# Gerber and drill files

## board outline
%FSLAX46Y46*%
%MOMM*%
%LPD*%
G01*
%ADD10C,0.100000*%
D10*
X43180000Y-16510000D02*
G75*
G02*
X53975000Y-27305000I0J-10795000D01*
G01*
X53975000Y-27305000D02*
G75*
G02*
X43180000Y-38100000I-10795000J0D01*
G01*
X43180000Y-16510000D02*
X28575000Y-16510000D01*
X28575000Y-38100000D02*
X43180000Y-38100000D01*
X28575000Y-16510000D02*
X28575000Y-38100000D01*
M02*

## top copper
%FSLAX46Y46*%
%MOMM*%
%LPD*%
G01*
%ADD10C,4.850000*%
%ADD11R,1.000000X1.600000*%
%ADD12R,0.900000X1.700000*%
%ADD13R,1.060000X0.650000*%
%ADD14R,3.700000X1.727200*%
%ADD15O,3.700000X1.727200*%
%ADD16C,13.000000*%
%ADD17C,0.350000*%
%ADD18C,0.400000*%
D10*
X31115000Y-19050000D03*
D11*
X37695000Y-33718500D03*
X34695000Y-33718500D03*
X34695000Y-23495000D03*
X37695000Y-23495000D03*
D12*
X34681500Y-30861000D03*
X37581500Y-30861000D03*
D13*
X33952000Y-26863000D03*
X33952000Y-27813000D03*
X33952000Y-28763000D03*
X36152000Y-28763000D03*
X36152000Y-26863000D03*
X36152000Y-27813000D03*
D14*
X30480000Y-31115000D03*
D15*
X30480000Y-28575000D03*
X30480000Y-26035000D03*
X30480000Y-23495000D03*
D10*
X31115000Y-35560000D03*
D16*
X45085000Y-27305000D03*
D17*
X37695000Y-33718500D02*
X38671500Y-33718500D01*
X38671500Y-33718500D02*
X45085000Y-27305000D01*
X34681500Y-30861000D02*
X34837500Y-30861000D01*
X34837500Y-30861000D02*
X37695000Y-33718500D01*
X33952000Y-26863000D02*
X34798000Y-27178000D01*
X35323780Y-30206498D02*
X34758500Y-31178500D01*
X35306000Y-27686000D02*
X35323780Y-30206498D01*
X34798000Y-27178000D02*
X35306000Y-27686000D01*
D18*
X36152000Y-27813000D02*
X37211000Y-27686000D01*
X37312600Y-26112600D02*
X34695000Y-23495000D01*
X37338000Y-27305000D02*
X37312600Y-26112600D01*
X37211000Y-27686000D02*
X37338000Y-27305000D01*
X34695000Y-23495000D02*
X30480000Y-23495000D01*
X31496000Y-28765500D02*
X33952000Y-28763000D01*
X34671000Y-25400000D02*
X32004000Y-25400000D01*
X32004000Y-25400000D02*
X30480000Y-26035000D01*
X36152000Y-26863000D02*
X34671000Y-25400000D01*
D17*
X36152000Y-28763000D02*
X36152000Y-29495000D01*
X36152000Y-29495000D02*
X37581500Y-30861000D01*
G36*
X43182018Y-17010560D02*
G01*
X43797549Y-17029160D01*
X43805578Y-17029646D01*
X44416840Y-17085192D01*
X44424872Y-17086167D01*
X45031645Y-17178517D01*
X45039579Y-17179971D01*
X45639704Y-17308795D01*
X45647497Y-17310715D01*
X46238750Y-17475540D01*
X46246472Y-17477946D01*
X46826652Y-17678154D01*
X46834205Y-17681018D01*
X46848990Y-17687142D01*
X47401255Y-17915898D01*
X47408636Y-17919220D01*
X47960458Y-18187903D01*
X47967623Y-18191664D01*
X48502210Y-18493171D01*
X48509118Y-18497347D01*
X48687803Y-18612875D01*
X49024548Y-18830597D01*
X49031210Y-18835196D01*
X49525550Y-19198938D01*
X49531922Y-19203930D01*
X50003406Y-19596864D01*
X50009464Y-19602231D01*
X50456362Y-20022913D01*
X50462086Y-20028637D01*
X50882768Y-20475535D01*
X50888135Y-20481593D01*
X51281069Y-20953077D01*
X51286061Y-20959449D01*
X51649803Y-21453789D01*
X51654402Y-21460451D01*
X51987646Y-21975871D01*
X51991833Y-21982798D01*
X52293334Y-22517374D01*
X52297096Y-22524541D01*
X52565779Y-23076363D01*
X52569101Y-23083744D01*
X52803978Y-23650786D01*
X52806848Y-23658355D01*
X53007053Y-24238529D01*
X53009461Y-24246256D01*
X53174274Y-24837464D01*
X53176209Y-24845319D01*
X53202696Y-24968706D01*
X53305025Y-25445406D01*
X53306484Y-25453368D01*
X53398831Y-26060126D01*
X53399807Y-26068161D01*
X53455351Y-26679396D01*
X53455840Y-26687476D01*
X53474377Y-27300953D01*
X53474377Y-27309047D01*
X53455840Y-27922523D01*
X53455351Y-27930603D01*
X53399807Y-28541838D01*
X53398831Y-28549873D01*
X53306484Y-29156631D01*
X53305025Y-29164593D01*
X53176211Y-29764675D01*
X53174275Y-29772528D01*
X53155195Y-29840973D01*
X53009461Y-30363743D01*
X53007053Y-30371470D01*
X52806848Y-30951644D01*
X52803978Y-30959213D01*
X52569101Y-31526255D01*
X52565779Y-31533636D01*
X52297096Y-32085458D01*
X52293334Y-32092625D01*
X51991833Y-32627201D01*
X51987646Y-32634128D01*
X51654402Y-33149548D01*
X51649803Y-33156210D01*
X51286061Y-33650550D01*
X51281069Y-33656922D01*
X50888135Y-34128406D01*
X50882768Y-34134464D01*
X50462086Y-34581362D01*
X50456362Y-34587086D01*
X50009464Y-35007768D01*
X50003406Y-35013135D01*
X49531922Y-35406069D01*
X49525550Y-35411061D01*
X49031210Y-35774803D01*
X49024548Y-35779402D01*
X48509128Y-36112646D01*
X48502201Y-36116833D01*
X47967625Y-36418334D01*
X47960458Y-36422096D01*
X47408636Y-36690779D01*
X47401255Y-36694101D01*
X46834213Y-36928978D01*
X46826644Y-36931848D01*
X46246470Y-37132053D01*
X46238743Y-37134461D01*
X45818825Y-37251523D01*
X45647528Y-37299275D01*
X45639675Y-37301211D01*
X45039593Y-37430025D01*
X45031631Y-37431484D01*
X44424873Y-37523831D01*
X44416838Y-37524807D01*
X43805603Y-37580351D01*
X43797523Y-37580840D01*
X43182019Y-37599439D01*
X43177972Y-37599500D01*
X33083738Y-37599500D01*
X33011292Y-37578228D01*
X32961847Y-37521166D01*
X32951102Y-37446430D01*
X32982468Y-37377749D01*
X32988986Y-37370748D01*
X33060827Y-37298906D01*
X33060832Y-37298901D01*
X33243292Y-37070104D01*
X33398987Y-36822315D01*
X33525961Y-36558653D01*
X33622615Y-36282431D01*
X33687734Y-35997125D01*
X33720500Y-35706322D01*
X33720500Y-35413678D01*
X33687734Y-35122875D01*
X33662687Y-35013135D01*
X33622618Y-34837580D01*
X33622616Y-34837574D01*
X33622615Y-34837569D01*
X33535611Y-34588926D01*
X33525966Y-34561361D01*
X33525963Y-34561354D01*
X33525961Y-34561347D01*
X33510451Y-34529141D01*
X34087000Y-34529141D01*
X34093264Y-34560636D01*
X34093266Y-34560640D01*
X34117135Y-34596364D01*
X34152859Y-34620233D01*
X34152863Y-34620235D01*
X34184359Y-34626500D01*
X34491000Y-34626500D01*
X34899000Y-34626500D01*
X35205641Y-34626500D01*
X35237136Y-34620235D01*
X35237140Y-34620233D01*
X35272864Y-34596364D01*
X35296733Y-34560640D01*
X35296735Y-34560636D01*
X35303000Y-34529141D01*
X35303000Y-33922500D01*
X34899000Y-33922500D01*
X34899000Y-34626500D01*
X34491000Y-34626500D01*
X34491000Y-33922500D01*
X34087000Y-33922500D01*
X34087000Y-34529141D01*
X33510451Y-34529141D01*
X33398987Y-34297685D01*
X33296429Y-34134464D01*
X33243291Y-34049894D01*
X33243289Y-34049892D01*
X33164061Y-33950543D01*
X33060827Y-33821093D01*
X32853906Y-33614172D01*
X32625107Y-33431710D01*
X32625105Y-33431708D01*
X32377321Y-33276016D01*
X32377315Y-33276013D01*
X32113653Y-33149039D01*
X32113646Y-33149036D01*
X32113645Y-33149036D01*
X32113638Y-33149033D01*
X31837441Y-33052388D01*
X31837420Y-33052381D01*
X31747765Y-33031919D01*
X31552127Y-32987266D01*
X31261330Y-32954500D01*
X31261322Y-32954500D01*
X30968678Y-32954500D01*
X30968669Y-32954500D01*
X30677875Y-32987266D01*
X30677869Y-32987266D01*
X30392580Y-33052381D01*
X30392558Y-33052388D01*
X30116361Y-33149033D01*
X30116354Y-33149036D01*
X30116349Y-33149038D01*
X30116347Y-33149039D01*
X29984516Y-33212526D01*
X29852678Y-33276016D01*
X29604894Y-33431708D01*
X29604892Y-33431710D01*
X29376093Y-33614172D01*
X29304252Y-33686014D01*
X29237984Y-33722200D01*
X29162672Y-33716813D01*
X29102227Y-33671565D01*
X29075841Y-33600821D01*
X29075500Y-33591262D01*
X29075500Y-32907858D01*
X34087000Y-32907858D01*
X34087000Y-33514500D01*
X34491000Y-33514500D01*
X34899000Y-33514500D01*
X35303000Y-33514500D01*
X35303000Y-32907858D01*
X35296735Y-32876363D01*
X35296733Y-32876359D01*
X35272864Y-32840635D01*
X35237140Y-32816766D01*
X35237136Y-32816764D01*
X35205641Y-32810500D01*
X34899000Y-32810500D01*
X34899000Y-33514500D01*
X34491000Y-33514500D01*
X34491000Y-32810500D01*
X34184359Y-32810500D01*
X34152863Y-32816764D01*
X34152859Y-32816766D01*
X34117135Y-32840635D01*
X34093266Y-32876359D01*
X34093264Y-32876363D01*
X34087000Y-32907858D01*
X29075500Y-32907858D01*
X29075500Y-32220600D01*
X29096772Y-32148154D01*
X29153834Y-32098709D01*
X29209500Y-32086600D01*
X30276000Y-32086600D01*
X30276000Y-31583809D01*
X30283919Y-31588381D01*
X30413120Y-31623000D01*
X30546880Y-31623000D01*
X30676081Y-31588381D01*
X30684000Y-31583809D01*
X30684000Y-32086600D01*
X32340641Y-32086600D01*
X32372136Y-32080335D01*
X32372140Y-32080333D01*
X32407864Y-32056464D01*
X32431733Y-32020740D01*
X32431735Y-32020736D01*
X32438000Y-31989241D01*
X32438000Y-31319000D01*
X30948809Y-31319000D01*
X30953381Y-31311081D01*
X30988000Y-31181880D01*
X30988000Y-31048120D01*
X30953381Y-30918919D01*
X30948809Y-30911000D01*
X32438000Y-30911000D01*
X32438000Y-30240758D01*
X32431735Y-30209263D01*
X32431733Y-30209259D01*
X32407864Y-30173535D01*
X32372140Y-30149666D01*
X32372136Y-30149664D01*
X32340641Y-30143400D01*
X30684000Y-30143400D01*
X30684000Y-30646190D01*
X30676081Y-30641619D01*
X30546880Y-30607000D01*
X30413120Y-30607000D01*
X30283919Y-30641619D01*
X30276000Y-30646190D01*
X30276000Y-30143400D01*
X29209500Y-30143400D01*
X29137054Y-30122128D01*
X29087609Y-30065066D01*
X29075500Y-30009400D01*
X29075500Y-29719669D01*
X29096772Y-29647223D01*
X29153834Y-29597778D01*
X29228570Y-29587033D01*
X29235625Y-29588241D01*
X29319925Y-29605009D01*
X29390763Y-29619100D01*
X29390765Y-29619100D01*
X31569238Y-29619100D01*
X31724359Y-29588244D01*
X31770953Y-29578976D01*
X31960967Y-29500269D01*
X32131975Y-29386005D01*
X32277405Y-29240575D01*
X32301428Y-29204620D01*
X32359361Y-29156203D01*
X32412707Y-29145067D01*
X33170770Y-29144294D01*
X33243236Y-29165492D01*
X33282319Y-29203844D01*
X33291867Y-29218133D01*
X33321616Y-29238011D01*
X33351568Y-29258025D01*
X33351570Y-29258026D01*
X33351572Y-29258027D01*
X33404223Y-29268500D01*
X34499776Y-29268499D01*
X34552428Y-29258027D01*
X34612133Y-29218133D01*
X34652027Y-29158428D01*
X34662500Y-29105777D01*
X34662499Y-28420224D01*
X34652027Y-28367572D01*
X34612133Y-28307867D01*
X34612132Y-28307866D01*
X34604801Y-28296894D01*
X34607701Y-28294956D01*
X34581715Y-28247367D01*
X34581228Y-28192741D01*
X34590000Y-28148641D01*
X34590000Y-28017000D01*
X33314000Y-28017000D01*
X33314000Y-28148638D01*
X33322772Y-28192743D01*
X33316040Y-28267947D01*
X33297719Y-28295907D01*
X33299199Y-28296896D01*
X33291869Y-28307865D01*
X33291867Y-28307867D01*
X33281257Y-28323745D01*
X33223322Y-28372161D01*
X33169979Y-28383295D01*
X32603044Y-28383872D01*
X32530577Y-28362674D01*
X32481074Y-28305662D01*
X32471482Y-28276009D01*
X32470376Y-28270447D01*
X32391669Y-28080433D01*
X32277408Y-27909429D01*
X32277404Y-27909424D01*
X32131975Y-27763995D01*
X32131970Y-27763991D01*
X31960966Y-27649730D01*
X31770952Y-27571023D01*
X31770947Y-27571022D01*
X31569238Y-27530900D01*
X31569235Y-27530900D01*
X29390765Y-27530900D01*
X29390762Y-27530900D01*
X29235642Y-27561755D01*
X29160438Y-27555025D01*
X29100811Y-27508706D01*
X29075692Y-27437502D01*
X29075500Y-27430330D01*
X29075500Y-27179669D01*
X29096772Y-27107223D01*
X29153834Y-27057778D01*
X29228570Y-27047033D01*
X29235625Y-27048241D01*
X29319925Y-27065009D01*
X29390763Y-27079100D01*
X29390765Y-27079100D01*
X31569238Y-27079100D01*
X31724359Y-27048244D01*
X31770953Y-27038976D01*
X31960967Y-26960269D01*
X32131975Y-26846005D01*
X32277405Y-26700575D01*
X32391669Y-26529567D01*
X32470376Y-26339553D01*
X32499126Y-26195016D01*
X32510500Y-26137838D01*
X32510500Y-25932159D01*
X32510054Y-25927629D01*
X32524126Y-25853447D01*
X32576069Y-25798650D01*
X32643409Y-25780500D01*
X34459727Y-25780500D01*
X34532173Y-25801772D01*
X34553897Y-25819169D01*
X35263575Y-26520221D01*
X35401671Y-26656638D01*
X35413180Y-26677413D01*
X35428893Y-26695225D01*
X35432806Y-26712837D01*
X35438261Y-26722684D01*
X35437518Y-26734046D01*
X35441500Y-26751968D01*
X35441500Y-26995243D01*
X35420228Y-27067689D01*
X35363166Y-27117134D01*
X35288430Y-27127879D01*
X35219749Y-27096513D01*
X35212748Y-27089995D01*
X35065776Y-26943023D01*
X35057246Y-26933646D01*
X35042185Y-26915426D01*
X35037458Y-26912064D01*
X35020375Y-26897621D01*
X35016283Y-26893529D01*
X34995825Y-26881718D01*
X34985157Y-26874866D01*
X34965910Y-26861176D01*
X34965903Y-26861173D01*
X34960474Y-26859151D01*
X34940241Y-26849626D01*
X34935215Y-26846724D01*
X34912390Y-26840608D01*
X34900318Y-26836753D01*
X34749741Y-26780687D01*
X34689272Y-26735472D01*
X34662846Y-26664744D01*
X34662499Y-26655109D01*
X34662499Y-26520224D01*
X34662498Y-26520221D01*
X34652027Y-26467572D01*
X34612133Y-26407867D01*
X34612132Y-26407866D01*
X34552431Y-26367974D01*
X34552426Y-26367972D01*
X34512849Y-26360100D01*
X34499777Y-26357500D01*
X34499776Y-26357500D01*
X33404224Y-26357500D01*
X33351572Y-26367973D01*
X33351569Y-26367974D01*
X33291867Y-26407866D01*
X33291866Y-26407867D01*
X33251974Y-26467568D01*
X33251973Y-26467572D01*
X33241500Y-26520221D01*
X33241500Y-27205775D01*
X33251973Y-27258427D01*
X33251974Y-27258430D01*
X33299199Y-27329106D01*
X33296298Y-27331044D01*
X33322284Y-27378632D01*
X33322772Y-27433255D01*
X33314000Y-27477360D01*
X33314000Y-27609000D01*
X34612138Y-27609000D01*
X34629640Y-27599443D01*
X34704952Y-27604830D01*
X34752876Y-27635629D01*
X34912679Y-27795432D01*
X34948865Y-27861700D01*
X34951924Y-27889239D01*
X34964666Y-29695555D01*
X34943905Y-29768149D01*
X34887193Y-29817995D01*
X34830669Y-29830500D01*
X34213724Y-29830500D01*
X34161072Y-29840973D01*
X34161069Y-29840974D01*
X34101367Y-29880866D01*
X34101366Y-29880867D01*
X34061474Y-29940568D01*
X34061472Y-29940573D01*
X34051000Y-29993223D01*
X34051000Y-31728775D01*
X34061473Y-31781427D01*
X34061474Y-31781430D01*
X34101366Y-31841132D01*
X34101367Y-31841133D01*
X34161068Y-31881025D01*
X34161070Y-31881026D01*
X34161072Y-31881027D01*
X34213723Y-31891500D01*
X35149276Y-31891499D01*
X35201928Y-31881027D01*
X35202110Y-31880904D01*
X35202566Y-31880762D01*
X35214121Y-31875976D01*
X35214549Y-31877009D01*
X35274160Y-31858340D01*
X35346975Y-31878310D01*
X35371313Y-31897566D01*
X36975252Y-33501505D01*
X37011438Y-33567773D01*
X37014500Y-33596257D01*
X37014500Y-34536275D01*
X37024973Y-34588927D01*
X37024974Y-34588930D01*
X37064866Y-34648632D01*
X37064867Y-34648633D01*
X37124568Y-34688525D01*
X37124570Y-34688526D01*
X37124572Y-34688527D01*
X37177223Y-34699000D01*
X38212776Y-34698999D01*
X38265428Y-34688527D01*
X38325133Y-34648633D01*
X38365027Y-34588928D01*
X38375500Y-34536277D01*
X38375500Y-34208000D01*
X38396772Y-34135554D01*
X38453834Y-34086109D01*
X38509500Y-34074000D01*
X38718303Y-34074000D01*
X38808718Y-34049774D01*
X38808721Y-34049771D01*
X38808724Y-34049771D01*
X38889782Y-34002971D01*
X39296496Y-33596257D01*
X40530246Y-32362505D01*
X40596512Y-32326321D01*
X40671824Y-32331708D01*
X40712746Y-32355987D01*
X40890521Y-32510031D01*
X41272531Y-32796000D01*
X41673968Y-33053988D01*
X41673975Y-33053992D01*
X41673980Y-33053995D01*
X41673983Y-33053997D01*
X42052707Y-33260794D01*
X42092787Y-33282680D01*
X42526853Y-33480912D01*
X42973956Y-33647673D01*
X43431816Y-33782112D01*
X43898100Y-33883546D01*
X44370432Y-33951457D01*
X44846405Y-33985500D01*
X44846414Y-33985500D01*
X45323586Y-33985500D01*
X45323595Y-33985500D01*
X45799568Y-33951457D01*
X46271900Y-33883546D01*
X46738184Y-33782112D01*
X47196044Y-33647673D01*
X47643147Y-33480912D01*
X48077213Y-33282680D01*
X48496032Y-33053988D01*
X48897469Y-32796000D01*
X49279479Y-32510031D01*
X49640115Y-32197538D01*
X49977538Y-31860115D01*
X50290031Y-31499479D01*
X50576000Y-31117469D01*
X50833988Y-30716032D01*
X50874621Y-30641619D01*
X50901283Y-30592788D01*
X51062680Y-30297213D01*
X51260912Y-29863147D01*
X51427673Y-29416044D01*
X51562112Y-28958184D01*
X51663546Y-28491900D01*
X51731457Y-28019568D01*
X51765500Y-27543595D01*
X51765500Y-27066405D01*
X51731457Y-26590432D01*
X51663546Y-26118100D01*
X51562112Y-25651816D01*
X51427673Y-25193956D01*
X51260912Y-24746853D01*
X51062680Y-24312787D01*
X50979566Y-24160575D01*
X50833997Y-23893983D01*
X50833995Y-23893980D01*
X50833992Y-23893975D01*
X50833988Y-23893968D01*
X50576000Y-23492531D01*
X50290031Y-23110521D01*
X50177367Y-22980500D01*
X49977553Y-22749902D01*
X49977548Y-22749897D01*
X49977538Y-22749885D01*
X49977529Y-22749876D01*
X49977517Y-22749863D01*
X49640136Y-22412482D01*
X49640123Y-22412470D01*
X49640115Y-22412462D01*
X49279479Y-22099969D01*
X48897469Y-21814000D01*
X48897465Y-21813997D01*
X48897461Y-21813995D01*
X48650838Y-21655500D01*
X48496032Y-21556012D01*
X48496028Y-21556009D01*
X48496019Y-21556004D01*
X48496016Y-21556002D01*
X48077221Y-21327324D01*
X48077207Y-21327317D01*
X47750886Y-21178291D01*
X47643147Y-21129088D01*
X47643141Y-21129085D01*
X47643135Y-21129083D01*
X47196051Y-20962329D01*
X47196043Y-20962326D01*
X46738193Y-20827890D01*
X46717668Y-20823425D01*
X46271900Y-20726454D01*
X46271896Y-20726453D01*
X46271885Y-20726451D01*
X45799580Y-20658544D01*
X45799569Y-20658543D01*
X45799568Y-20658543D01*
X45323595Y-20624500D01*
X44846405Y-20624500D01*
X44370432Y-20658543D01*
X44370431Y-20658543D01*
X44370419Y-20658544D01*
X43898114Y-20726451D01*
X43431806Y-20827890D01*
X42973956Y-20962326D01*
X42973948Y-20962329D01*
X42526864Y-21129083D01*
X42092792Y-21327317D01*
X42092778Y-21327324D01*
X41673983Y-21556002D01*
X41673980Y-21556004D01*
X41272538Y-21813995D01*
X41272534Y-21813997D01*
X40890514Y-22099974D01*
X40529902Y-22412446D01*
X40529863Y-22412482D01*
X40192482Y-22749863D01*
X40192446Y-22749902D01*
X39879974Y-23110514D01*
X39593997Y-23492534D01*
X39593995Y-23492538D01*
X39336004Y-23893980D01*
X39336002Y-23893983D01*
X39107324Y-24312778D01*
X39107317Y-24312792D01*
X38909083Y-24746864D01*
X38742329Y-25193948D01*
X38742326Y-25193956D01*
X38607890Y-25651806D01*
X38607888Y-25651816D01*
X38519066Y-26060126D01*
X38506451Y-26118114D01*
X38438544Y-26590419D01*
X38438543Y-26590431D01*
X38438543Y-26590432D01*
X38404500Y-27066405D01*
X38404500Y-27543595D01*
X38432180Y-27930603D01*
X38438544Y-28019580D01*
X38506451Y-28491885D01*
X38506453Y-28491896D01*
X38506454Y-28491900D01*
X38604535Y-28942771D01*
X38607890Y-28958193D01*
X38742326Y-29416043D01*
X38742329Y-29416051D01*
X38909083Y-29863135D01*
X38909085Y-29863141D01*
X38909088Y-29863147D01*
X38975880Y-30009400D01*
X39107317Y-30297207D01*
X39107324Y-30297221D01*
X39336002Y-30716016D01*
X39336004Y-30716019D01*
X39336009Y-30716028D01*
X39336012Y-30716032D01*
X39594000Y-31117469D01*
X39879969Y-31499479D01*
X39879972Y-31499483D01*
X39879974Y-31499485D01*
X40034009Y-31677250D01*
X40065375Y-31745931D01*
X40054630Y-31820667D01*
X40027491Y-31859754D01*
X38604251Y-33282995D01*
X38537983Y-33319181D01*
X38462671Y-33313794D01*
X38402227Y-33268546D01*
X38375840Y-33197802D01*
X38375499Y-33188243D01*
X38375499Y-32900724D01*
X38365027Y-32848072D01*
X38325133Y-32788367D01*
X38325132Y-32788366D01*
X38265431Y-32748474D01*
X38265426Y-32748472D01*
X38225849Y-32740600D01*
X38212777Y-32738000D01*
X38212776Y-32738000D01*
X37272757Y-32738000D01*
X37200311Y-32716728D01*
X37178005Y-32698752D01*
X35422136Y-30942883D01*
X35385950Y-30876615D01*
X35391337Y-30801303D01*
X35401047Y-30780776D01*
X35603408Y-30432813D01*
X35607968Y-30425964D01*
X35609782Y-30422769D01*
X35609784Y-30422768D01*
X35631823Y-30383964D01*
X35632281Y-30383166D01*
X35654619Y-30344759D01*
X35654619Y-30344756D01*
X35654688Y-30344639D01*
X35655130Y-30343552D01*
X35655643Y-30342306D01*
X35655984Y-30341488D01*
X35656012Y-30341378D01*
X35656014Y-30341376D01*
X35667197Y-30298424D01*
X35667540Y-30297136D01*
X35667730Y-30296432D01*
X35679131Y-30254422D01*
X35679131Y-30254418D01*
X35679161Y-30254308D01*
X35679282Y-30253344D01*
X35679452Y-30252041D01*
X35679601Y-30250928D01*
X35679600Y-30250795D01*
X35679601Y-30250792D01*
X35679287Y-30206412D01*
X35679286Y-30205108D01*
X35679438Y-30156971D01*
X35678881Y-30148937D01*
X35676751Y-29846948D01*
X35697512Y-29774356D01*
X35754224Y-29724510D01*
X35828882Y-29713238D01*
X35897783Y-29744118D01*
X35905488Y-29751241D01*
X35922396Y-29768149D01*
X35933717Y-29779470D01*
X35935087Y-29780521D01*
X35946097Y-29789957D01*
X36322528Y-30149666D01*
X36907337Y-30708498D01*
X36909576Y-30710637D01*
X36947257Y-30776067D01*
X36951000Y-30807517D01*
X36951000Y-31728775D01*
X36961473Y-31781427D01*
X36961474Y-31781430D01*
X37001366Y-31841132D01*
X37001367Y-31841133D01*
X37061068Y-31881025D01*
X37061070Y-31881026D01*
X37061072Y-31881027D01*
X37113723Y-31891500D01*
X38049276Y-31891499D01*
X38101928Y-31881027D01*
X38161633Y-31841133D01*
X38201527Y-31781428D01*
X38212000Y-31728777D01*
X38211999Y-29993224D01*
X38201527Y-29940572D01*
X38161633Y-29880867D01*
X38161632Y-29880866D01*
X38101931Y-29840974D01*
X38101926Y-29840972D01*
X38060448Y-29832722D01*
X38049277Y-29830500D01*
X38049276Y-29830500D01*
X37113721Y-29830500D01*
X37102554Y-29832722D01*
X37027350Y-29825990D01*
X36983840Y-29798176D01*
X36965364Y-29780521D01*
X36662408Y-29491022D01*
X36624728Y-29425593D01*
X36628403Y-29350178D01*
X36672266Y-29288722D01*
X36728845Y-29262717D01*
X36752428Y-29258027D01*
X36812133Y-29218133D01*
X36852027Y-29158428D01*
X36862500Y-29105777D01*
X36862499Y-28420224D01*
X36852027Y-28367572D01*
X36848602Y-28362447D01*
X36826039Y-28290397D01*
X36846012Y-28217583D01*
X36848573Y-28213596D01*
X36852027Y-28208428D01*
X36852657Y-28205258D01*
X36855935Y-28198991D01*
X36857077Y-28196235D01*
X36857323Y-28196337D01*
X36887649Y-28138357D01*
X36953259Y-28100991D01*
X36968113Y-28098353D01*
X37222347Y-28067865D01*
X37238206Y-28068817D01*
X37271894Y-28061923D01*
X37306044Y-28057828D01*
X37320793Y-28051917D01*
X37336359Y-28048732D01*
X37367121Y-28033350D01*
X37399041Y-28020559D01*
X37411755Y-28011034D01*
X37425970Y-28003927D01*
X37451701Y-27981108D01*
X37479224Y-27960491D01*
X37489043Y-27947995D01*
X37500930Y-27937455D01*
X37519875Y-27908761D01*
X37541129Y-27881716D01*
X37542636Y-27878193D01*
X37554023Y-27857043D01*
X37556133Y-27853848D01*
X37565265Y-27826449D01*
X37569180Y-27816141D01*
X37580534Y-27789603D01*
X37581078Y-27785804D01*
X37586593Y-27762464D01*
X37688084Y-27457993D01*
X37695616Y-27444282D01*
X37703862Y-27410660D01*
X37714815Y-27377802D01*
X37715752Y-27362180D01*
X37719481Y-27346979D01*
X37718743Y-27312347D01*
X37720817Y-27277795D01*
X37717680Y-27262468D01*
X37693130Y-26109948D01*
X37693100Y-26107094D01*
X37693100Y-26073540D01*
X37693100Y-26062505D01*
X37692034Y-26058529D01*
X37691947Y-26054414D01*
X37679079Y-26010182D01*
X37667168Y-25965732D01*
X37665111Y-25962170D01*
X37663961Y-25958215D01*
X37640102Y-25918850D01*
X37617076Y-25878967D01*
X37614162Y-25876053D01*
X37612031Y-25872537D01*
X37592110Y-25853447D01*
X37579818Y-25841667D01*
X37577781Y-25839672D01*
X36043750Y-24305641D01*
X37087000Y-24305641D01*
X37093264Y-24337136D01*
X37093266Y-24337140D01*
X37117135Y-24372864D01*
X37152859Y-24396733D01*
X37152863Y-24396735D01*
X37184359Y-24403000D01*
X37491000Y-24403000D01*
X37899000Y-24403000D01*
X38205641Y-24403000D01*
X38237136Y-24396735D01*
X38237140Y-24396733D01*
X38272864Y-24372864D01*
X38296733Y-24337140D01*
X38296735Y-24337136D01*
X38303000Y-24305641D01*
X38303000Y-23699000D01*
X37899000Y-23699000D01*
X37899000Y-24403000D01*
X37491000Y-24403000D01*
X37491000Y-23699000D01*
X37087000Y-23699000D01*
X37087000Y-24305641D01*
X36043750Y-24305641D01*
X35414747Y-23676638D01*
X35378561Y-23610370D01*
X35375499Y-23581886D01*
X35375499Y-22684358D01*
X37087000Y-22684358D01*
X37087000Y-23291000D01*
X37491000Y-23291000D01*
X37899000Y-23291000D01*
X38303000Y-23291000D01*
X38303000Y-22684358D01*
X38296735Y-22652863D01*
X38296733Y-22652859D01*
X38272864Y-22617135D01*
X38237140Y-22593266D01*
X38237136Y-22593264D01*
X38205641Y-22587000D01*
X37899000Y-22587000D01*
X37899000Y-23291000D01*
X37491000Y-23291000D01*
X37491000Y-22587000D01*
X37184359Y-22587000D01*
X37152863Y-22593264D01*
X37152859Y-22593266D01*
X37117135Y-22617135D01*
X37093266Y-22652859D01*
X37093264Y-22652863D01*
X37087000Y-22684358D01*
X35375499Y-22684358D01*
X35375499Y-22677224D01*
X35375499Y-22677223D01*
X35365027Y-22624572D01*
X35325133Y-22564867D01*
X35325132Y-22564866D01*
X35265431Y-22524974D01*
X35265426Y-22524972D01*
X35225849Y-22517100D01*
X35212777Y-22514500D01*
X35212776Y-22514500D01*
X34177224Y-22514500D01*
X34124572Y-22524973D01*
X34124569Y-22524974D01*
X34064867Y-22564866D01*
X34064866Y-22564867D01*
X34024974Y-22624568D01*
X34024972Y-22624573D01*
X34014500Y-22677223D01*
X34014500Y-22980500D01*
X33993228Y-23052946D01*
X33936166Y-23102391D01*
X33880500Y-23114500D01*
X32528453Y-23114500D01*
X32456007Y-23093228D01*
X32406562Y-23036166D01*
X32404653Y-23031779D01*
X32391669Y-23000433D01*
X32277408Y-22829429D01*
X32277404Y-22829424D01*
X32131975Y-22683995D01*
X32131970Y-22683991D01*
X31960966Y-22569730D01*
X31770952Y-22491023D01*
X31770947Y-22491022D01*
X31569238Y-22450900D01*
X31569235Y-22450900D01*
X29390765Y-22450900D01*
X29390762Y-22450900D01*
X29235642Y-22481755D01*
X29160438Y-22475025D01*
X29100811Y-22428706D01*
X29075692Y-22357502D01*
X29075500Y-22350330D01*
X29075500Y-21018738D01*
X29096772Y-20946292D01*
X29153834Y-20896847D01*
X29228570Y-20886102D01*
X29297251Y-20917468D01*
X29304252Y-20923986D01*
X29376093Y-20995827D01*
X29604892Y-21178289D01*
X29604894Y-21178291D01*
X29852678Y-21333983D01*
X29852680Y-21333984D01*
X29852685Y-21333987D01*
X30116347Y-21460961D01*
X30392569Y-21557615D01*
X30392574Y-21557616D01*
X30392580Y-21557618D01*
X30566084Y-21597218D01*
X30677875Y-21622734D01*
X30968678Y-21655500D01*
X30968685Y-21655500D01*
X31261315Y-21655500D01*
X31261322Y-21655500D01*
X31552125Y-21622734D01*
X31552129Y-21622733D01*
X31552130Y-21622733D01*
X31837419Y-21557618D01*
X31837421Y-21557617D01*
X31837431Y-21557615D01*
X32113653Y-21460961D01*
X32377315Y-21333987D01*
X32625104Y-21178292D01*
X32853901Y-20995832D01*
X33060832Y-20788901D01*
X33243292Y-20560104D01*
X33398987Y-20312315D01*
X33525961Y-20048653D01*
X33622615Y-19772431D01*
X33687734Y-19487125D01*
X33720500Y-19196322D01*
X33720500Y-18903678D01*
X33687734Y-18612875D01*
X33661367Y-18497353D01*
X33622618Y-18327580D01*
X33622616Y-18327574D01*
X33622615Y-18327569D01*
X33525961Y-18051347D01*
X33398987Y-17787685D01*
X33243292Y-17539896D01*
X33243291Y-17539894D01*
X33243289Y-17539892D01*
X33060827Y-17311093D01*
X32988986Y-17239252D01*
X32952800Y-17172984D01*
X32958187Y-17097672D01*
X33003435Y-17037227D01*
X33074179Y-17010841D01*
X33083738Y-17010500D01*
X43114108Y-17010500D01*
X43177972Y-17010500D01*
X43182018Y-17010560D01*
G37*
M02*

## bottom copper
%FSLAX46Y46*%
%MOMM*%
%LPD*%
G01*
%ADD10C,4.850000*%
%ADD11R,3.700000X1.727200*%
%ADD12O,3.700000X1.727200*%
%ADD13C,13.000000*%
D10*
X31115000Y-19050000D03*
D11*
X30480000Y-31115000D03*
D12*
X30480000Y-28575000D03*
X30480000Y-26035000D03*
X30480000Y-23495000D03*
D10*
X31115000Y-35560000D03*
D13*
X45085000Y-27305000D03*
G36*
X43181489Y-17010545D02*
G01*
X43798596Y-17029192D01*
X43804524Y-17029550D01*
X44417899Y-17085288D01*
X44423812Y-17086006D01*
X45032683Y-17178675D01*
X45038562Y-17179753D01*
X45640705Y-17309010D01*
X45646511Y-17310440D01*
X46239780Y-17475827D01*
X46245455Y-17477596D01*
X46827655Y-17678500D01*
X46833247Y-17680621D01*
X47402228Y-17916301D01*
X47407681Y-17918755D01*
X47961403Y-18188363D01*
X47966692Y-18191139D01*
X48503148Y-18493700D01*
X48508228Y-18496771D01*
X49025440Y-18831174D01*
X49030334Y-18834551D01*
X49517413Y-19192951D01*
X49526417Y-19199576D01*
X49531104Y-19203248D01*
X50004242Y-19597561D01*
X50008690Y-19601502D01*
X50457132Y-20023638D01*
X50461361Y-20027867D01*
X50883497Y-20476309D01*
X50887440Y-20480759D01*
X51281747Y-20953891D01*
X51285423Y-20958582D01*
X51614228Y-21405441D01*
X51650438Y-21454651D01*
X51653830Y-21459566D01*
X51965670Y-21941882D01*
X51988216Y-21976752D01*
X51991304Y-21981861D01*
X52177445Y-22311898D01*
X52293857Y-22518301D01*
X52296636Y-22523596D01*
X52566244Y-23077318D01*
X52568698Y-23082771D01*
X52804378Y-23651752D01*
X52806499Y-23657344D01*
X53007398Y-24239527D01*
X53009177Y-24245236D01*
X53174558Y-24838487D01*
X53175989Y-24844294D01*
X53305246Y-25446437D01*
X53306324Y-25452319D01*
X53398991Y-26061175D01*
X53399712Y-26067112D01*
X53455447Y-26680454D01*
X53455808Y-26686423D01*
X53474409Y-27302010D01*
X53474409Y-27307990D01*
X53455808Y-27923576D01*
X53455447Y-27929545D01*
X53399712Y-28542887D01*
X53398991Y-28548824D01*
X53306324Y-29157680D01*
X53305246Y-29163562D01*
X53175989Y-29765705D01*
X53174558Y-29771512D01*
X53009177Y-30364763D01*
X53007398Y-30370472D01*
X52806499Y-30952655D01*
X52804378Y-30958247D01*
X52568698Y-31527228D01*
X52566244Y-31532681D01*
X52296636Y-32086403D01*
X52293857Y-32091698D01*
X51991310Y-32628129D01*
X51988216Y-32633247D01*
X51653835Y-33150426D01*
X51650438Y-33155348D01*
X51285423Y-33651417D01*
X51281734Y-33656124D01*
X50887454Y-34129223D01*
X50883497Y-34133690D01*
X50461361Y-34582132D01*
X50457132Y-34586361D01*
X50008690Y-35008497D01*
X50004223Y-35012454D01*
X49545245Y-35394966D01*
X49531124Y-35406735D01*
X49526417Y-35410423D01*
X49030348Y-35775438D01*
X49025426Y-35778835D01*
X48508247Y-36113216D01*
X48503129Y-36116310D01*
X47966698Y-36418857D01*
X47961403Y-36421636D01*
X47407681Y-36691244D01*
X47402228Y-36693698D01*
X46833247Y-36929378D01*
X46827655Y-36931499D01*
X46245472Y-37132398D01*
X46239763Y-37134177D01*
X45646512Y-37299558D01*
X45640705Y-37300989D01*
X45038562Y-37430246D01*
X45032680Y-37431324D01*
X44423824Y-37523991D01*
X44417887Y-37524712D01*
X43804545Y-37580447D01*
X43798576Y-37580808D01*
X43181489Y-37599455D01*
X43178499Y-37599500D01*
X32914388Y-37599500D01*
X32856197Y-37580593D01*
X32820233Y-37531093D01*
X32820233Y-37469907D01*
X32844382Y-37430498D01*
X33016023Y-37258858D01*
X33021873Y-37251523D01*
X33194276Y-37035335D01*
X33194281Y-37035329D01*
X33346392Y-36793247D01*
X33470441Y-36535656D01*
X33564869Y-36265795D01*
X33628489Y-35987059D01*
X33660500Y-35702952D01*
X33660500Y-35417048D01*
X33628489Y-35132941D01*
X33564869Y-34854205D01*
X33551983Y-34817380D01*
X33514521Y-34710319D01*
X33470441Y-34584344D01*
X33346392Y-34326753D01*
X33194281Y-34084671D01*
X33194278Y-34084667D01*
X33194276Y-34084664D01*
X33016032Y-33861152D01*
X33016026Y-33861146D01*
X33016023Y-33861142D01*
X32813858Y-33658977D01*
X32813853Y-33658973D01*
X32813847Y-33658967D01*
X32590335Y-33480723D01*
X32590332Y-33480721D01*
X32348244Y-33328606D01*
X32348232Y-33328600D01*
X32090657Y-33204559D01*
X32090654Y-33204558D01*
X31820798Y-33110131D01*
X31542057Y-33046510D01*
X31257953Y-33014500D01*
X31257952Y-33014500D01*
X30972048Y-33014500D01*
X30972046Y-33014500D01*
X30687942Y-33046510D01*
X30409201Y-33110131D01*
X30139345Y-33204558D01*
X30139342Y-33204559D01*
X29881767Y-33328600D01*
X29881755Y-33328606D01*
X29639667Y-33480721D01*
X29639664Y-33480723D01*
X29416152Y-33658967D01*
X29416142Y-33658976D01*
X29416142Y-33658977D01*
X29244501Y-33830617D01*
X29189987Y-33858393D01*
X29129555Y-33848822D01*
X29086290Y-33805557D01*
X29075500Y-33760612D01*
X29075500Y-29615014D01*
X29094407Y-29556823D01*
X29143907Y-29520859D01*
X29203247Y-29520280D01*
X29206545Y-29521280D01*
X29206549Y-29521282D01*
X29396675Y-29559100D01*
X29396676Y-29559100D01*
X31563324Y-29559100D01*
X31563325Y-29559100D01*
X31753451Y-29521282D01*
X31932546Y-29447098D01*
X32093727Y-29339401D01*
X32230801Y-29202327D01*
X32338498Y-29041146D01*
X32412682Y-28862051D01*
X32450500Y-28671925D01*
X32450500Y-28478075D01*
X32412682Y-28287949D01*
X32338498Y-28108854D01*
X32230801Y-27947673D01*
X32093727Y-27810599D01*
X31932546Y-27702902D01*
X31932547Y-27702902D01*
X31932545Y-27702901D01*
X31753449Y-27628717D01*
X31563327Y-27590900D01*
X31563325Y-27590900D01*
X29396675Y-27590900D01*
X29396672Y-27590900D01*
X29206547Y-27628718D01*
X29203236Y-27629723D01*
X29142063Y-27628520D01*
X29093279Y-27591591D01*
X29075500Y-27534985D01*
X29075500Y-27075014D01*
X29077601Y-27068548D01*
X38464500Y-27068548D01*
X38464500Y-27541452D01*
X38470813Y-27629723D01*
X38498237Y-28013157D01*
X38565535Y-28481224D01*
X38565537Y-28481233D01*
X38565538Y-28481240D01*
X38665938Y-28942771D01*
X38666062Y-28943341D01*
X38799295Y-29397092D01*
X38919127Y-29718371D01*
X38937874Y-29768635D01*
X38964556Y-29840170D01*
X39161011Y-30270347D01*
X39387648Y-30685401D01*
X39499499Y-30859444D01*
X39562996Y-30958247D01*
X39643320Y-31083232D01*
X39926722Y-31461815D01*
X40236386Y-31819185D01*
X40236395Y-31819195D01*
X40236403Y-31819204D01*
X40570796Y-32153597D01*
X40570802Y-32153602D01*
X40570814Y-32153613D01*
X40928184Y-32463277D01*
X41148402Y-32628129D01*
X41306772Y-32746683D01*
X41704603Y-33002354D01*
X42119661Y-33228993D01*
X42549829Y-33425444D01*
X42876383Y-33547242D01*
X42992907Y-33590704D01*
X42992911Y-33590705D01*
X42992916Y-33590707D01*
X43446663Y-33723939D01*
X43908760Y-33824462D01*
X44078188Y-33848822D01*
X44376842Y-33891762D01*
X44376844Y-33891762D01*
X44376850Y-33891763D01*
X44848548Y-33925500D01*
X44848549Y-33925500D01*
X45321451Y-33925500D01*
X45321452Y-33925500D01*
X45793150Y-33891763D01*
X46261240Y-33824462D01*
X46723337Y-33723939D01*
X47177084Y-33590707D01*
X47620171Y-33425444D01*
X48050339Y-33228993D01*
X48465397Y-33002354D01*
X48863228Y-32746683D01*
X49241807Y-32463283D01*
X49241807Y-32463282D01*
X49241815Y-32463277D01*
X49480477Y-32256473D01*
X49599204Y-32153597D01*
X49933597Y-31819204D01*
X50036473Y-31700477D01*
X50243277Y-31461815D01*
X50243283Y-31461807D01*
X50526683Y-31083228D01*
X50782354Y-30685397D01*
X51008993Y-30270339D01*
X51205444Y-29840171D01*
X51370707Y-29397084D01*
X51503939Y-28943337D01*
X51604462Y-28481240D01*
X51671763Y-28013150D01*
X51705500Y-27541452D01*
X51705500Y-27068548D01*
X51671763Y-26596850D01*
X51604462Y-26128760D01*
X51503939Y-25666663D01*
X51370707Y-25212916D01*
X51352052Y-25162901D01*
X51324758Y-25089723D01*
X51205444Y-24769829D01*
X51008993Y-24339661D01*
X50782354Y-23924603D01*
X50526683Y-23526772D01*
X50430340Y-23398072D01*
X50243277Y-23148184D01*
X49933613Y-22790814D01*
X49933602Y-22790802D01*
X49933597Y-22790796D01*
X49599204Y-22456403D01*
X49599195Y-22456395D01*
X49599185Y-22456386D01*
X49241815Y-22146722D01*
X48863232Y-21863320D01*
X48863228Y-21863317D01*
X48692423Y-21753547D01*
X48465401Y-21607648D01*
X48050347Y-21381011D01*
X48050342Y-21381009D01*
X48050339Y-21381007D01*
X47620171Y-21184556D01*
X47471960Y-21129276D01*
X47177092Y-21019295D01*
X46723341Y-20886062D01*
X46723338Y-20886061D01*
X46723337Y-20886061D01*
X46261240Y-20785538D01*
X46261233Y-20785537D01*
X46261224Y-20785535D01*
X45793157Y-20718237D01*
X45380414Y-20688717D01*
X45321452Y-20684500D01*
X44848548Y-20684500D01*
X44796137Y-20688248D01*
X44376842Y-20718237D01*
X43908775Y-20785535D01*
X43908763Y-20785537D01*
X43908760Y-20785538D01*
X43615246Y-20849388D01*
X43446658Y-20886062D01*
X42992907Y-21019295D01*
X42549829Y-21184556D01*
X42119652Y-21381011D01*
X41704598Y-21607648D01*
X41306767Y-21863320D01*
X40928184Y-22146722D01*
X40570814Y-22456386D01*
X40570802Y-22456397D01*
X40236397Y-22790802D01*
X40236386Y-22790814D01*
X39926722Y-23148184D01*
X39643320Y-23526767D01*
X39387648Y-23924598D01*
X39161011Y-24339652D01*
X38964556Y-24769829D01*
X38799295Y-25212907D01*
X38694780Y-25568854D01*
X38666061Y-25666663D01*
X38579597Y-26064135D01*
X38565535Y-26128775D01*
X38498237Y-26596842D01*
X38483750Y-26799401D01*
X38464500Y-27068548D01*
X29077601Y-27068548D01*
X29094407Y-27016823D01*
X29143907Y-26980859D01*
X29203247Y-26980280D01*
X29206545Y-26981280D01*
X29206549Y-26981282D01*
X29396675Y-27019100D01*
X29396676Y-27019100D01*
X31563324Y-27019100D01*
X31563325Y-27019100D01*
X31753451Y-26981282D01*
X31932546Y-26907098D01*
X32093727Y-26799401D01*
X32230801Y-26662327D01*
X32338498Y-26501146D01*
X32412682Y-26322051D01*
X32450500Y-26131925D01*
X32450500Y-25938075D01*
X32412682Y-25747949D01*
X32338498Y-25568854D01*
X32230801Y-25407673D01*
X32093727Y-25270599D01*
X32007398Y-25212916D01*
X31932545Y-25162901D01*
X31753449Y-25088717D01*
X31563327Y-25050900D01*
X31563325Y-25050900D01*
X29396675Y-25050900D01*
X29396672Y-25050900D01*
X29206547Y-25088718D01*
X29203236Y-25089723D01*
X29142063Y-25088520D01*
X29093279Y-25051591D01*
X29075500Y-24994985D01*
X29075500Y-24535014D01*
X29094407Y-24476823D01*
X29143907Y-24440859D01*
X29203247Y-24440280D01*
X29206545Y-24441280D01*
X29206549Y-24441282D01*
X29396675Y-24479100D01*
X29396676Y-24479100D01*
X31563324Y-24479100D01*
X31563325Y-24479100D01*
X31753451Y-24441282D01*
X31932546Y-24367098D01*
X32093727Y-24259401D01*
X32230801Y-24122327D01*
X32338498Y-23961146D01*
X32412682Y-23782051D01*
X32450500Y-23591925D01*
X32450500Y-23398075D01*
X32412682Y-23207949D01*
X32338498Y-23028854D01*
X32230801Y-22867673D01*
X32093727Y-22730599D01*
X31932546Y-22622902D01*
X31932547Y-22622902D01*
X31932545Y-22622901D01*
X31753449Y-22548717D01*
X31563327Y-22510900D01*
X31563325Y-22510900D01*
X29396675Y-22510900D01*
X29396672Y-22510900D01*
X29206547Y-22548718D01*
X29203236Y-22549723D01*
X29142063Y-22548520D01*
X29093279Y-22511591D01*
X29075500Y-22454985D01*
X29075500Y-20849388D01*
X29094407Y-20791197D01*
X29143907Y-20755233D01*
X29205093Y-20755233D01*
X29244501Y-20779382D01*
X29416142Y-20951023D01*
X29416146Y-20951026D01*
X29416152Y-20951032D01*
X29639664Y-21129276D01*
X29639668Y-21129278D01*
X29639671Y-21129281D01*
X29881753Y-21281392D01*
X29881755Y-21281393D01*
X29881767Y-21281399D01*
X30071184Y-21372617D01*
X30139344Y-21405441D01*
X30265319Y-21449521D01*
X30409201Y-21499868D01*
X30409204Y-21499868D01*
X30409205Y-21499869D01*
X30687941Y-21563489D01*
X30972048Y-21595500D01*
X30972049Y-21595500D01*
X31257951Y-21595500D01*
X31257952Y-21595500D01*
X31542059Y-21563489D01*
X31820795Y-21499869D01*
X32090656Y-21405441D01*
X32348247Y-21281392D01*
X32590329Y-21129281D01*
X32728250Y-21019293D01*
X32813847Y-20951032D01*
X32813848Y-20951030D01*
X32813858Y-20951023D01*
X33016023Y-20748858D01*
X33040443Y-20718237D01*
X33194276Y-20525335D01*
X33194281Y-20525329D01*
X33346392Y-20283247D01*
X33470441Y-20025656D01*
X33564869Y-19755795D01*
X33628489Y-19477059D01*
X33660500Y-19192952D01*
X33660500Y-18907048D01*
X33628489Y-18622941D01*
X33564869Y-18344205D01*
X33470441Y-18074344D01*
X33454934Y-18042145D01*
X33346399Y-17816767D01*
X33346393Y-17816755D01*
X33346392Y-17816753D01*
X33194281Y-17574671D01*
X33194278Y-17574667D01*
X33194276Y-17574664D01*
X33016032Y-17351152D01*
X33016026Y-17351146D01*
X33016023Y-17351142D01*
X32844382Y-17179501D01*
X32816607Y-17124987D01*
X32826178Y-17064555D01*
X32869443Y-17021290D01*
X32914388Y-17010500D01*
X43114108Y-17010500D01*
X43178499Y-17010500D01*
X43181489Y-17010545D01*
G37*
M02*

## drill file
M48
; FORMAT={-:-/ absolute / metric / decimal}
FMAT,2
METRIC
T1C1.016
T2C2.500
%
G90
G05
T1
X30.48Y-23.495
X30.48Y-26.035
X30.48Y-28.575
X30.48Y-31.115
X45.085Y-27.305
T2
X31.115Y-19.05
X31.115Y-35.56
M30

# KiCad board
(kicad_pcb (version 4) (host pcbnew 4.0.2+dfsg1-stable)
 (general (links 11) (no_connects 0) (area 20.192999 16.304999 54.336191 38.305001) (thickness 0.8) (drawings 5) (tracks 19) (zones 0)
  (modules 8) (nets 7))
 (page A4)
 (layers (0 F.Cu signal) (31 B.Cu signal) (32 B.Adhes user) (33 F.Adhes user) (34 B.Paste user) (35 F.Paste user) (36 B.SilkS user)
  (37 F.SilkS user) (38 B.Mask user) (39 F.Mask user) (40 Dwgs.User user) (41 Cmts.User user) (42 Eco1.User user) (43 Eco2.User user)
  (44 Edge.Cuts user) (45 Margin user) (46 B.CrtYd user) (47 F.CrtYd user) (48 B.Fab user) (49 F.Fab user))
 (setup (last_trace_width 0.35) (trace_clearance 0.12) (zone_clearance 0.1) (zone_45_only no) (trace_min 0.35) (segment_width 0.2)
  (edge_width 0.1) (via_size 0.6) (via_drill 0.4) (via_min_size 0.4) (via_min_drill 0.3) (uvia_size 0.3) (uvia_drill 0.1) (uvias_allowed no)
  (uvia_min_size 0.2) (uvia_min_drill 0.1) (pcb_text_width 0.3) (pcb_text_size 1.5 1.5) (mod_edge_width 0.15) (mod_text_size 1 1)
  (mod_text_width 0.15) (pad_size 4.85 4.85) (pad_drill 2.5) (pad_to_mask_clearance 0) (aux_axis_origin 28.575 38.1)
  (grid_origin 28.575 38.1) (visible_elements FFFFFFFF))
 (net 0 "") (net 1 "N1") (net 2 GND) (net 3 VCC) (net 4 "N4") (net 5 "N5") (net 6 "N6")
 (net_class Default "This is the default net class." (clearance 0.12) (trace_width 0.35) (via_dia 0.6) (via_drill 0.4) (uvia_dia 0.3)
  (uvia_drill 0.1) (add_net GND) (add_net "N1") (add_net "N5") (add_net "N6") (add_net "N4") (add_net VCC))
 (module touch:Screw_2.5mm (layer F.Cu) (at 31.115 19.05)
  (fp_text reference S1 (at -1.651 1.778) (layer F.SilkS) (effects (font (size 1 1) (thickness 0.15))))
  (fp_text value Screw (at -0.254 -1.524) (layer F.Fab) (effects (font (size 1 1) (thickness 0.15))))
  (pad 1 thru_hole circle (at 0 0) (size 4.85 4.85) (drill 2.5) (layers *.Cu *.Mask F.SilkS)))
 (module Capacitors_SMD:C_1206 (layer F.Cu) (at 36.195 33.7185 180)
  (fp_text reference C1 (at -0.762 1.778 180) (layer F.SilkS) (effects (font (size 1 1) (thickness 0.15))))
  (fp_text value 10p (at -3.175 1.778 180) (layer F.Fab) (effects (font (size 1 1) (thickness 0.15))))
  (pad 1 smd rect (at -1.5 0 180) (size 1 1.6) (layers F.Cu F.Paste F.Mask) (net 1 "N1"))
  (pad 2 smd rect (at 1.5 0 180) (size 1 1.6) (layers F.Cu F.Paste F.Mask) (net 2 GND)))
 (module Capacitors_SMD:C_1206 (layer F.Cu) (at 36.195 23.495)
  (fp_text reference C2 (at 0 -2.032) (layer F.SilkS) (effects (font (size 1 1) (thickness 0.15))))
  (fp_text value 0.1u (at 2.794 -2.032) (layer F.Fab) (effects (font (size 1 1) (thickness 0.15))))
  (pad 1 smd rect (at -1.5 0) (size 1 1.6) (layers F.Cu F.Paste F.Mask) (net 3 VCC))
  (pad 2 smd rect (at 1.5 0) (size 1 1.6) (layers F.Cu F.Paste F.Mask) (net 2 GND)))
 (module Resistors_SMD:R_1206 (layer F.Cu) (at 36.1315 30.861)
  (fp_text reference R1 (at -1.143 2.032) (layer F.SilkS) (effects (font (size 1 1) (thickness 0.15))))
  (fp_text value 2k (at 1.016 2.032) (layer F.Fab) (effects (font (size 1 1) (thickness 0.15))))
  (pad 1 smd rect (at -1.45 0) (size 0.9 1.7) (layers F.Cu F.Paste F.Mask) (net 1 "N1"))
  (pad 2 smd rect (at 1.45 0) (size 0.9 1.7) (layers F.Cu F.Paste F.Mask) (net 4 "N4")))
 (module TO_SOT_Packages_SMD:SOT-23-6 (layer F.Cu) (at 35.052 27.813)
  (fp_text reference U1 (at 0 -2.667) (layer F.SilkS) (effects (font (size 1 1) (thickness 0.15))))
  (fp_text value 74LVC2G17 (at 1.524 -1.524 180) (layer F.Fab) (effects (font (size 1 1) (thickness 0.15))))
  (pad 1 smd rect (at -1.1 -0.95) (size 1.06 0.65) (layers F.Cu F.Paste F.Mask) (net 1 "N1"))
  (pad 2 smd rect (at -1.1 0) (size 1.06 0.65) (layers F.Cu F.Paste F.Mask) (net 2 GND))
  (pad 3 smd rect (at -1.1 0.95) (size 1.06 0.65) (layers F.Cu F.Paste F.Mask) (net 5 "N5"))
  (pad 4 smd rect (at 1.1 0.95) (size 1.06 0.65) (layers F.Cu F.Paste F.Mask) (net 4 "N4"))
  (pad 6 smd rect (at 1.1 -0.95) (size 1.06 0.65) (layers F.Cu F.Paste F.Mask) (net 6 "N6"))
  (pad 5 smd rect (at 1.1 0) (size 1.06 0.65) (layers F.Cu F.Paste F.Mask) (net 3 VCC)))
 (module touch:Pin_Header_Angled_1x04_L (layer F.Cu) (at 30.48 31.115 180)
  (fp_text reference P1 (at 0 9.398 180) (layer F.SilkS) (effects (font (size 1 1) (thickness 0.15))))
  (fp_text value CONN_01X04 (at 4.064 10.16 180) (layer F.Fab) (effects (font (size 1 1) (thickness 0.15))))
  (pad 1 thru_hole rect (at 0 0 180) (size 3.7 1.7272) (drill 1.016) (layers *.Cu *.Mask F.SilkS) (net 2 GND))
  (pad 2 thru_hole oval (at 0 2.54 180) (size 3.7 1.7272) (drill 1.016) (layers *.Cu *.Mask F.SilkS) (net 5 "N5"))
  (pad 3 thru_hole oval (at 0 5.08 180) (size 3.7 1.7272) (drill 1.016) (layers *.Cu *.Mask F.SilkS) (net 6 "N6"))
  (pad 4 thru_hole oval (at 0 7.62 180) (size 3.7 1.7272) (drill 1.016) (layers *.Cu *.Mask F.SilkS) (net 3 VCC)))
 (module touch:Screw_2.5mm (layer F.Cu) (at 31.115 35.56)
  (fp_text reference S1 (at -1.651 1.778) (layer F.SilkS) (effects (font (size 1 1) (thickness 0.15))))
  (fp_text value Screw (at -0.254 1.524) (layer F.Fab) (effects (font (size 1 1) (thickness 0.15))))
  (pad 1 thru_hole circle (at 0 0) (size 4.85 4.85) (drill 2.5) (layers *.Cu *.Mask F.SilkS)))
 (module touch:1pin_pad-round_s (layer F.Cu) (at 45.085 27.305)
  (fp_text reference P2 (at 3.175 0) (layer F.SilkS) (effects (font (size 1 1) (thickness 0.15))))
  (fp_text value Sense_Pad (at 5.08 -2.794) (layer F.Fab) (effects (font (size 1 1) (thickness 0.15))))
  (pad 1 thru_hole circle (at 0 0) (size 13 13) (drill 1.016) (layers *.Cu *.Mask F.SilkS) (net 1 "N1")))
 (gr_arc (start 43.18 27.305) (end 43.18 16.51) (angle 90) (layer Edge.Cuts) (width 0.1))
 (gr_arc (start 43.18 27.305) (end 53.975 27.305) (angle 90) (layer Edge.Cuts) (width 0.1))
 (gr_line (start 43.18 16.51) (end 28.575 16.51) (angle 90) (layer Edge.Cuts) (width 0.1))
 (gr_line (start 28.575 38.1) (end 43.18 38.1) (angle 90) (layer Edge.Cuts) (width 0.1))
 (gr_line (start 28.575 16.51) (end 28.575 38.1) (angle 90) (layer Edge.Cuts) (width 0.1))
 (segment (start 37.695 33.7185) (end 38.6715 33.7185) (width 0.35) (layer F.Cu) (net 1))
 (segment (start 38.6715 33.7185) (end 45.085 27.305) (width 0.35) (layer F.Cu) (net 1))
 (segment (start 34.6815 30.861) (end 34.8375 30.861) (width 0.35) (layer F.Cu) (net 1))
 (segment (start 34.8375 30.861) (end 37.695 33.7185) (width 0.35) (layer F.Cu) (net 1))
 (segment (start 33.952 26.863) (end 34.798 27.178) (width 0.35) (layer F.Cu) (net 1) (status 10))
 (segment (start 35.32378 30.206498) (end 34.7585 31.1785) (width 0.35) (layer F.Cu) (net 1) (status 20))
 (segment (start 35.306 27.686) (end 35.32378 30.206498) (width 0.35) (layer F.Cu) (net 1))
 (segment (start 34.798 27.178) (end 35.306 27.686) (width 0.35) (layer F.Cu) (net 1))
 (segment (start 36.152 27.813) (end 37.211 27.686) (width 0.4) (layer F.Cu) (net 3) (status 10))
 (segment (start 37.3126 26.1126) (end 34.695 23.495) (width 0.4) (layer F.Cu) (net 3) (status 20))
 (segment (start 37.338 27.305) (end 37.3126 26.1126) (width 0.4) (layer F.Cu) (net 3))
 (segment (start 37.211 27.686) (end 37.338 27.305) (width 0.4) (layer F.Cu) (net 3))
 (segment (start 34.695 23.495) (end 30.48 23.495) (width 0.4) (layer F.Cu) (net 3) (status 10))
 (segment (start 31.496 28.7655) (end 33.952 28.763) (width 0.4) (layer F.Cu) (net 5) (status 20))
 (segment (start 34.671 25.4) (end 32.004 25.4) (width 0.4) (layer F.Cu) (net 6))
 (segment (start 32.004 25.4) (end 30.48 26.035) (width 0.4) (layer F.Cu) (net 6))
 (segment (start 36.152 26.863) (end 34.671 25.4) (width 0.4) (layer F.Cu) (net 6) (status 10))
 (segment (start 36.152 28.763) (end 36.152 29.495) (width 0.35) (layer F.Cu) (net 4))
 (segment (start 36.152 29.495) (end 37.5815 30.861) (width 0.35) (layer F.Cu) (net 4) (status 20))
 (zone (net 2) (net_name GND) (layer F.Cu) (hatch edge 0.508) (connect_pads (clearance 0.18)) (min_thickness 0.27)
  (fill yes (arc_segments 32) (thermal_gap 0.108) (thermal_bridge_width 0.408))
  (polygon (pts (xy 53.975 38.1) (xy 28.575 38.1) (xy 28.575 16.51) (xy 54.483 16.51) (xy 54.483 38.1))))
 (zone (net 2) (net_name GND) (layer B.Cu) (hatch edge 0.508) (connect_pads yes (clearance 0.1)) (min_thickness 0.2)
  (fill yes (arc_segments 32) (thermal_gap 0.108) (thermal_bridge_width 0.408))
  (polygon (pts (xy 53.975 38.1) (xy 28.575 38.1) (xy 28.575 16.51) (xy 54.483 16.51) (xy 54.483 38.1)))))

